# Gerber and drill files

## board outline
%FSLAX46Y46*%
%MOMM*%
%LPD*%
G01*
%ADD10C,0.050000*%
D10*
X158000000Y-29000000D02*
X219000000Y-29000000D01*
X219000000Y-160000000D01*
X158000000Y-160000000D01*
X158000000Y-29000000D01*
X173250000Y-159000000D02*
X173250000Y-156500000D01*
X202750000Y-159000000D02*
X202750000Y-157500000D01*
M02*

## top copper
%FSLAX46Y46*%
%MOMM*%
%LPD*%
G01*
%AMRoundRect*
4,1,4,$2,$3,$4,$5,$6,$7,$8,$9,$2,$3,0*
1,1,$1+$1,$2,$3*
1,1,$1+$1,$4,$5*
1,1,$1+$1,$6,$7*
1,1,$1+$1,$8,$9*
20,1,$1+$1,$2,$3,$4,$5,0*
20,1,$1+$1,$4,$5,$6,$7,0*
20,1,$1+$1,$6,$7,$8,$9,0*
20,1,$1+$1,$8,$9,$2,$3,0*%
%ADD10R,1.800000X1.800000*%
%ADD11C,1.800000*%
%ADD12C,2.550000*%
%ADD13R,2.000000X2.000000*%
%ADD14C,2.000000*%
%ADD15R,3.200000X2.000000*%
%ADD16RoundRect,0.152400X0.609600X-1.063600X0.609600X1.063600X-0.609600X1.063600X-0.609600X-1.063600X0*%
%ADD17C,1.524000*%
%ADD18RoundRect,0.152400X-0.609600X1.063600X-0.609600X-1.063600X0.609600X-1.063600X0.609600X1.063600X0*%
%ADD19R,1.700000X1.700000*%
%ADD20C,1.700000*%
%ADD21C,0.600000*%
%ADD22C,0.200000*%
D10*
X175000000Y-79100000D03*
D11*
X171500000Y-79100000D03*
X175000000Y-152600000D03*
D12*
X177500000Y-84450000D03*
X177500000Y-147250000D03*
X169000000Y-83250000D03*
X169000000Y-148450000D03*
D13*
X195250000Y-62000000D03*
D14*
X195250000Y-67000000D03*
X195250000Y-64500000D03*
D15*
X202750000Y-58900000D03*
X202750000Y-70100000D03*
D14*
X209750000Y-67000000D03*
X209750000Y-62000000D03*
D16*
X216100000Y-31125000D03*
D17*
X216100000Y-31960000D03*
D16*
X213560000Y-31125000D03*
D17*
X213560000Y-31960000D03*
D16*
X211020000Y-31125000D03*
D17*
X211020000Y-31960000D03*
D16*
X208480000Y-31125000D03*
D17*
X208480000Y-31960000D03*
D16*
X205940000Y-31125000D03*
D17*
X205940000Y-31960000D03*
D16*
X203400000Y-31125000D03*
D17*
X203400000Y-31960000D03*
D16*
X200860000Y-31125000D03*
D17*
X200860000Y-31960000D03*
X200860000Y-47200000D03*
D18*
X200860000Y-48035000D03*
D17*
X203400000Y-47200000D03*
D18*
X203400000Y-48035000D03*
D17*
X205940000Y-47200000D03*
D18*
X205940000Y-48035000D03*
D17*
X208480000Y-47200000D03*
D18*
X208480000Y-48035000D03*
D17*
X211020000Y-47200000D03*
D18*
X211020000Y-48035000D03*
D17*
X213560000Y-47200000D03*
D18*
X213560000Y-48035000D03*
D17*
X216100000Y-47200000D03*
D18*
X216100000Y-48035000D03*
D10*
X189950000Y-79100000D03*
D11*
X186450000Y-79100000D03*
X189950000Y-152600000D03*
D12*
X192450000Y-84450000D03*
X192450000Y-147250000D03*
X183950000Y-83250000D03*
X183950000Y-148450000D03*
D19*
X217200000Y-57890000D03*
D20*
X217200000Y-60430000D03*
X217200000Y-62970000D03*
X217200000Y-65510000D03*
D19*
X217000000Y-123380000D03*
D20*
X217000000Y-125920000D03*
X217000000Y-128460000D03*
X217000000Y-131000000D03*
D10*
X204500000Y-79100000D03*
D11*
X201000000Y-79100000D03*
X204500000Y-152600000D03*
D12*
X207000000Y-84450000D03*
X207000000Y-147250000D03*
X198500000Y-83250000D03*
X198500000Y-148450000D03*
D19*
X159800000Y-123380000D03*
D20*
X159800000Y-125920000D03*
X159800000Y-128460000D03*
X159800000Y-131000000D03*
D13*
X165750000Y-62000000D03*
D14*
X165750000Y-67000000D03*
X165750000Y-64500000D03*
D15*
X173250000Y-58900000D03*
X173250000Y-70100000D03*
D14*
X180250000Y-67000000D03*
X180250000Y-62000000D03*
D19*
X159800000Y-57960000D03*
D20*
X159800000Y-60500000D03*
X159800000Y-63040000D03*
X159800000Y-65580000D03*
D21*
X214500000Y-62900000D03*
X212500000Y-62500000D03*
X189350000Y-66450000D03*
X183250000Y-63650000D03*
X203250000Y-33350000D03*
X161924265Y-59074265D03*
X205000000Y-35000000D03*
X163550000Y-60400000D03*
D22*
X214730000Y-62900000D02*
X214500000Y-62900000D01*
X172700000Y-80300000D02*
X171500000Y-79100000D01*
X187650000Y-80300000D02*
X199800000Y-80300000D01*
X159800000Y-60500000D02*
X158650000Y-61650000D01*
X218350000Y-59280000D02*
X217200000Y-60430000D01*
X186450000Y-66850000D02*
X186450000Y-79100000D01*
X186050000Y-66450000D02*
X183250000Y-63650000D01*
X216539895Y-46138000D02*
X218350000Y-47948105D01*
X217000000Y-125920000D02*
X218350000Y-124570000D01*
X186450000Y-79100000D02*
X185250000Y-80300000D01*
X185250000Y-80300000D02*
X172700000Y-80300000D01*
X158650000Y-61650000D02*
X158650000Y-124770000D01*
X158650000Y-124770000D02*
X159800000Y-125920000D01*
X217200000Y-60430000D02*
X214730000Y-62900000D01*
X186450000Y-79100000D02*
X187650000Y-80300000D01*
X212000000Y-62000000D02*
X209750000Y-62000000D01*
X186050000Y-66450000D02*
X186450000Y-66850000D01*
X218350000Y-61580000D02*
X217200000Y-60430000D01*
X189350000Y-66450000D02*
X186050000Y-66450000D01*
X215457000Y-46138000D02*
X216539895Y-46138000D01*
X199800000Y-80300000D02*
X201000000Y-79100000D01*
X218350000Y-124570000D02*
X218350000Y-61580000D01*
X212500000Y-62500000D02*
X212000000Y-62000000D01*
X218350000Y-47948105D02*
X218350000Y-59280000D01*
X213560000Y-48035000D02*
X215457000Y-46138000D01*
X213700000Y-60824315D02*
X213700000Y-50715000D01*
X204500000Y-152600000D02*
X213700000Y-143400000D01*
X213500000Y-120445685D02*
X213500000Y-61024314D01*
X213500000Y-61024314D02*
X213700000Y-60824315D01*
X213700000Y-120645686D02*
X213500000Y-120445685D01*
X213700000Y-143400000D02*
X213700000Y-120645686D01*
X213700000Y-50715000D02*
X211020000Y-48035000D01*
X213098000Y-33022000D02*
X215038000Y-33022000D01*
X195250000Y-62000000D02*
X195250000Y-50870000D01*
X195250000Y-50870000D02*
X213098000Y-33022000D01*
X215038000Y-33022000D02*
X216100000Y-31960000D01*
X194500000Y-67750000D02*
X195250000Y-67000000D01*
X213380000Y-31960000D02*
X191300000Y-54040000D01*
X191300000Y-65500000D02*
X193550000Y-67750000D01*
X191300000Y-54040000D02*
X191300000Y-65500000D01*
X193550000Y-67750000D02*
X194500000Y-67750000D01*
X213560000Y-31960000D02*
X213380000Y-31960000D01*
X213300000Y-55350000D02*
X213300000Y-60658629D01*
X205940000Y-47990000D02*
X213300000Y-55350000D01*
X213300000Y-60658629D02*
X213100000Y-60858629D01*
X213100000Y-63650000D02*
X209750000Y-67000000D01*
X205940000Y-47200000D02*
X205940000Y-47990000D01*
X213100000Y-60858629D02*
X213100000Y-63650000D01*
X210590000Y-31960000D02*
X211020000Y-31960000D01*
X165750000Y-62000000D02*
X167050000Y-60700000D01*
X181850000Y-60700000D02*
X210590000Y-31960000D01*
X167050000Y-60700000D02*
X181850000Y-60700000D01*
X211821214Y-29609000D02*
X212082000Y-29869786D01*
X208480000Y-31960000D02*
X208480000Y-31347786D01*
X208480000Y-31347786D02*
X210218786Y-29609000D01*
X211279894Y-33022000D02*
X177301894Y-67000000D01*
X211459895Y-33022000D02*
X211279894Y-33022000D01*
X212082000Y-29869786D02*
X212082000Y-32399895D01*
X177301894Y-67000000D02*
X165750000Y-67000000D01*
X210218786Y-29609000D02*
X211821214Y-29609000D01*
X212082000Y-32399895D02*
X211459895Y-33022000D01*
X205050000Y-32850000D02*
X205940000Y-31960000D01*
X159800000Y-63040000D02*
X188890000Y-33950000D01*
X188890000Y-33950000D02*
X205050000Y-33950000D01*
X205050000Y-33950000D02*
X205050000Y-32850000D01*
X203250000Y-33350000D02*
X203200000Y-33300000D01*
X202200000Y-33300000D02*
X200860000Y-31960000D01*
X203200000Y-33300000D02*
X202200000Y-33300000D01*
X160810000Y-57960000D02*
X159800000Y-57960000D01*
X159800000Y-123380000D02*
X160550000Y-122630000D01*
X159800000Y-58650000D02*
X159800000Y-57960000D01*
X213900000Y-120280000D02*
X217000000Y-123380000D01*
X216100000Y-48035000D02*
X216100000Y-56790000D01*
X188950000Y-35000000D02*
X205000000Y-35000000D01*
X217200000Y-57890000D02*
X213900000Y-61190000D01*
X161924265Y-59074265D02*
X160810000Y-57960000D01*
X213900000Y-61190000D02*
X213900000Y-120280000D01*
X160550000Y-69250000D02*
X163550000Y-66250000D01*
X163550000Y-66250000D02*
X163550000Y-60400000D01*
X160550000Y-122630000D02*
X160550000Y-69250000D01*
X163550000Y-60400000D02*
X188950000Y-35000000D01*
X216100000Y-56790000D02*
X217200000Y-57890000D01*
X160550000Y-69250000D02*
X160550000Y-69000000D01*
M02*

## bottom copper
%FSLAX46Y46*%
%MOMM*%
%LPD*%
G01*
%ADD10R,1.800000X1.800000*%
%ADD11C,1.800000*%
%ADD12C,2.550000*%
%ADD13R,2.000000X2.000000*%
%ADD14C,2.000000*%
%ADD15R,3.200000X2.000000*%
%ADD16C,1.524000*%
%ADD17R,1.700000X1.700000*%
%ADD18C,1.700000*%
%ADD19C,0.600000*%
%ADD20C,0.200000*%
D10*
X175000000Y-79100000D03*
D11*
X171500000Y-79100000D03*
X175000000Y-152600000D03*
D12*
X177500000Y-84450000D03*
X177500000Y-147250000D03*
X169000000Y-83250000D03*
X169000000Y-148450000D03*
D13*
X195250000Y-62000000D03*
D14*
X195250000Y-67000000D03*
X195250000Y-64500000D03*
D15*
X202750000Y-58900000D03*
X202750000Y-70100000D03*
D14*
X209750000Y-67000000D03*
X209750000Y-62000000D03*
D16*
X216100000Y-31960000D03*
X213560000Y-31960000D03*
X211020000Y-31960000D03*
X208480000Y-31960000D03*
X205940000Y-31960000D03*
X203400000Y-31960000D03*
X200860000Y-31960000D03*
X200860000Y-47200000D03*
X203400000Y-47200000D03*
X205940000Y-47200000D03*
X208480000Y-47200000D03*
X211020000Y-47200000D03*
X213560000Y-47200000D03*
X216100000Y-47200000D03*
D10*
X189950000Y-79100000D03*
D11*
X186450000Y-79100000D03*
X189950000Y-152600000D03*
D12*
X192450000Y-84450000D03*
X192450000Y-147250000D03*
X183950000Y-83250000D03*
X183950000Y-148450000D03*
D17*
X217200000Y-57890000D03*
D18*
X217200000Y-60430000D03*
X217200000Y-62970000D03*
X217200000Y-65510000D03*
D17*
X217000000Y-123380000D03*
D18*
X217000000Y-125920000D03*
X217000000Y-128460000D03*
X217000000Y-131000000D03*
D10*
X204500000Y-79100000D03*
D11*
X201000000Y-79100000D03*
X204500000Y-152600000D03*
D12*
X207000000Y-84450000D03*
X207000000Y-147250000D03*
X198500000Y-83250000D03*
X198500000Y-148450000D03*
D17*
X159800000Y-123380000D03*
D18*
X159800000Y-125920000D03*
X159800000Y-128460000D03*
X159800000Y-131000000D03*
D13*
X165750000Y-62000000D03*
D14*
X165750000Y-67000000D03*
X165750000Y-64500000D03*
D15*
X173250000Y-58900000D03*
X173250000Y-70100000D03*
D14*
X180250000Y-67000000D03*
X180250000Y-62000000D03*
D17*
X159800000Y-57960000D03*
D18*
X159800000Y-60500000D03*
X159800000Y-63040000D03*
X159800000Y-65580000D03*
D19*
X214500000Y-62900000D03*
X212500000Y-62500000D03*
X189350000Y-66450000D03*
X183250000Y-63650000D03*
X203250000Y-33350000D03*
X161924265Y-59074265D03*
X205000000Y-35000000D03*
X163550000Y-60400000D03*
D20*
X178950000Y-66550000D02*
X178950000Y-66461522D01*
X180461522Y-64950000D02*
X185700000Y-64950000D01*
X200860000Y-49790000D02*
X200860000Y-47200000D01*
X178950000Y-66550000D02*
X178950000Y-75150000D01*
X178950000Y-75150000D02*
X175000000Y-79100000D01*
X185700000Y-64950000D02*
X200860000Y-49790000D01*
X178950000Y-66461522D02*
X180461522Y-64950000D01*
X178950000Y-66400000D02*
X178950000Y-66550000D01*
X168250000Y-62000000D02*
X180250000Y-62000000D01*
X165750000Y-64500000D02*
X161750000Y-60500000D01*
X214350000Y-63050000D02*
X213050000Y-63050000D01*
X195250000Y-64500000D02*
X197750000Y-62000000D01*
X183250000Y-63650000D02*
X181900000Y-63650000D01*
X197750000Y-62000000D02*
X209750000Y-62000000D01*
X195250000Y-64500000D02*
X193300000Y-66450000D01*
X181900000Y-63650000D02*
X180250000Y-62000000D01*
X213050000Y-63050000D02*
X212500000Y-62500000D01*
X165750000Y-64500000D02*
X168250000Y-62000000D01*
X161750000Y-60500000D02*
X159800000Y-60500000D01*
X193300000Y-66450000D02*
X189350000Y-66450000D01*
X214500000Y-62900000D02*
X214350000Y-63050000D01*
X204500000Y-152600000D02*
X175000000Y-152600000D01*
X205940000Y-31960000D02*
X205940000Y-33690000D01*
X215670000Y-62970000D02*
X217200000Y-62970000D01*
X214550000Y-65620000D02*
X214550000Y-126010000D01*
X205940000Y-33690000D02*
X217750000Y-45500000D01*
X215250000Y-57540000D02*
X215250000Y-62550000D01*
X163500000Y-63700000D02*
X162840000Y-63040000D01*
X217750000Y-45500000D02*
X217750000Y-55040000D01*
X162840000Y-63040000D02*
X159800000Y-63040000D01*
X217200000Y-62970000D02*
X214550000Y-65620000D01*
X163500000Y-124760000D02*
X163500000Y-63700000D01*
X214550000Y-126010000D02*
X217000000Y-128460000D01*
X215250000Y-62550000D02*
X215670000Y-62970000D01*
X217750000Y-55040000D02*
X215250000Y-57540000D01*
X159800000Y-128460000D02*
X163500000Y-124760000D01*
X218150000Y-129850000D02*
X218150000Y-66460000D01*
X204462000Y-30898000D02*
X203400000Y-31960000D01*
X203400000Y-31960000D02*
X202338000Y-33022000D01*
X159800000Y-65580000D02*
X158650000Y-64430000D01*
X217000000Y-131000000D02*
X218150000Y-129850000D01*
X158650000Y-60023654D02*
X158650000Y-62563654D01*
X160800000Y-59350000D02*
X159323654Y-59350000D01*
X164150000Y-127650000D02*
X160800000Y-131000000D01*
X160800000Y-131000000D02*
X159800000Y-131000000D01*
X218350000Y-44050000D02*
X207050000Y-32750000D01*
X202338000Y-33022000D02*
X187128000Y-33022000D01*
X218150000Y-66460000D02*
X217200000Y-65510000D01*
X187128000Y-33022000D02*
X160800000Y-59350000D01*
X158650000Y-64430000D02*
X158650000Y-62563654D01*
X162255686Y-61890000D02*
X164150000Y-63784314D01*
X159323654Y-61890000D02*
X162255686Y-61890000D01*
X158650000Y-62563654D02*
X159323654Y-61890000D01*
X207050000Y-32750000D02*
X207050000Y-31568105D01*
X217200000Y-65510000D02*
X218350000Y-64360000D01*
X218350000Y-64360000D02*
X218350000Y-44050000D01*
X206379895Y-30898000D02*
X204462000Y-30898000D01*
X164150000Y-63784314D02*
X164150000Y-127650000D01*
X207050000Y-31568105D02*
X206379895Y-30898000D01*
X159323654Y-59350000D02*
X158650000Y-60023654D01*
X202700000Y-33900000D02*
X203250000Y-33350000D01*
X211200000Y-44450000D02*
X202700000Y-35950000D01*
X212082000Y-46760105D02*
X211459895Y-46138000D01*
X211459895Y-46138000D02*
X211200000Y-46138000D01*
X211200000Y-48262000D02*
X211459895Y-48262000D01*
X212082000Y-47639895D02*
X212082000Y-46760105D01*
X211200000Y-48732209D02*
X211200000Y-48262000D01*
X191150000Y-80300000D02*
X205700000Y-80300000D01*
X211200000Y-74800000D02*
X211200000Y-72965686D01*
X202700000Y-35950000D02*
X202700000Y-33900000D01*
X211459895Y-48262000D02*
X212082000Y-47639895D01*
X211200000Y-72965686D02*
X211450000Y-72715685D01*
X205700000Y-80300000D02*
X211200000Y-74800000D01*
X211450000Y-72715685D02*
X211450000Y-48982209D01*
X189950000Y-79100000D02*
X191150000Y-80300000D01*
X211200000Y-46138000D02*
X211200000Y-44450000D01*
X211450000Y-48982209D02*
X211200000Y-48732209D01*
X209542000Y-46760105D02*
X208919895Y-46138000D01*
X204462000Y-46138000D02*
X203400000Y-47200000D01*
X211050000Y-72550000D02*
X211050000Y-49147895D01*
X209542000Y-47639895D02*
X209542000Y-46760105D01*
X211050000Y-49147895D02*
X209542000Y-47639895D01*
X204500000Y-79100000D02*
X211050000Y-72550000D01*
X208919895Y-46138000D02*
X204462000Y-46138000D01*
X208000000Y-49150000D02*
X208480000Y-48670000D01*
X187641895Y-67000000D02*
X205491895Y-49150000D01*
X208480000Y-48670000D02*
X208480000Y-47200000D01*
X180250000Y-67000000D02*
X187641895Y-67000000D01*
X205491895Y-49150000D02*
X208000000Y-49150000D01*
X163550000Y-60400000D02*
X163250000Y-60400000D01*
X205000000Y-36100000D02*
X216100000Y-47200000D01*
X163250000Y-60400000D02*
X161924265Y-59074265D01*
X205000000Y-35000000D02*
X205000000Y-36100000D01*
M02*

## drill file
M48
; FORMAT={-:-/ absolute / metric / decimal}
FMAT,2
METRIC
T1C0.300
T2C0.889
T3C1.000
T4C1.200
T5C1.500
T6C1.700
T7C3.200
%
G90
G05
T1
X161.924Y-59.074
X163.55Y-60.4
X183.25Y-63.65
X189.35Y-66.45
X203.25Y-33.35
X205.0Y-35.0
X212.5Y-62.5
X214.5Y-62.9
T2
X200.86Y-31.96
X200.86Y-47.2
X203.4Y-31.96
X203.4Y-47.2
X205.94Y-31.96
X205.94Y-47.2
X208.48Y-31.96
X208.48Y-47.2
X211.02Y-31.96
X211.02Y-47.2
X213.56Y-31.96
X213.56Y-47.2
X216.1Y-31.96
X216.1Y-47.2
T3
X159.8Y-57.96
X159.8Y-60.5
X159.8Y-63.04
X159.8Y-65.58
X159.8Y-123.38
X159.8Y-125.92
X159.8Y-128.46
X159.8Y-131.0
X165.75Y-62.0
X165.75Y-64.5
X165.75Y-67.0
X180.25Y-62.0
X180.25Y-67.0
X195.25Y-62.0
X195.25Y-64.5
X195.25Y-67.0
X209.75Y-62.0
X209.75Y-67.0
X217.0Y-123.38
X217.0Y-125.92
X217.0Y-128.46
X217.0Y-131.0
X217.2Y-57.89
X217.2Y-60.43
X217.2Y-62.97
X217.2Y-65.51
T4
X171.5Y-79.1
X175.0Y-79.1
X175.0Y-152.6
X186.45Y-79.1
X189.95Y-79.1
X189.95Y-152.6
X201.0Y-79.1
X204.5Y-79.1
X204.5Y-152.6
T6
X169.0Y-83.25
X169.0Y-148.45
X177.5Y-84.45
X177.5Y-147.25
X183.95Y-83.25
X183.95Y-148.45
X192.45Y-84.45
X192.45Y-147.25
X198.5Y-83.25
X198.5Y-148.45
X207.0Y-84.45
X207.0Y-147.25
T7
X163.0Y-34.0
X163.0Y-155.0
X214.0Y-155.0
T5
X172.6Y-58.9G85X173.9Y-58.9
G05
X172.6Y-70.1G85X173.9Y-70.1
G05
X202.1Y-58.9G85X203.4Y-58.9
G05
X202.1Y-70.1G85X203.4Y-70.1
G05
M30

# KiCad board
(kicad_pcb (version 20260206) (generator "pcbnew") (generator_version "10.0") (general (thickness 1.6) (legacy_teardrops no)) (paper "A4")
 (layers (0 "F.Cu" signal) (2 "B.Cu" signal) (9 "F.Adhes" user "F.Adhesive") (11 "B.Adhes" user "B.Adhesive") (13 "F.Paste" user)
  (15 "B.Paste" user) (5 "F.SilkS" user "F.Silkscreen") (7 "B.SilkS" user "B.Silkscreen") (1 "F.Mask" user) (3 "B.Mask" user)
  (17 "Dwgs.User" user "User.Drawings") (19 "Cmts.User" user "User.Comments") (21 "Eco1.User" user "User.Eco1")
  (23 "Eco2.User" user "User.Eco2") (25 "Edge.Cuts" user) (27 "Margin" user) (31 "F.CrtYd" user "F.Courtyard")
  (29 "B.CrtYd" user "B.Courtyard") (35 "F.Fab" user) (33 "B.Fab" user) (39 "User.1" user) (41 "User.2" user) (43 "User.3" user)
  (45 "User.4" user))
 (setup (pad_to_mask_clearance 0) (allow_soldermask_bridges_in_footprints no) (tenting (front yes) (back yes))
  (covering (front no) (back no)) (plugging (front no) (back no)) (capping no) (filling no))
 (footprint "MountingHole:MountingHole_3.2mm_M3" (layer "F.Cu") (at 163 34)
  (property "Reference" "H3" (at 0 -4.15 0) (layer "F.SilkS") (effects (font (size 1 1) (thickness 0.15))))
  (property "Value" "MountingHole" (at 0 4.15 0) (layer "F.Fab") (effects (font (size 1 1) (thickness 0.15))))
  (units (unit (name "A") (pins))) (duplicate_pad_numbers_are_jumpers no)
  (pad "" np_thru_hole circle (at 0 0) (size 3.2 3.2) (drill 3.2) (layers "*.Cu" "*.Mask")))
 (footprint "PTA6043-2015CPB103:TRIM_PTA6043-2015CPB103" (layer "F.Cu") (at 173.25 115.85 -90)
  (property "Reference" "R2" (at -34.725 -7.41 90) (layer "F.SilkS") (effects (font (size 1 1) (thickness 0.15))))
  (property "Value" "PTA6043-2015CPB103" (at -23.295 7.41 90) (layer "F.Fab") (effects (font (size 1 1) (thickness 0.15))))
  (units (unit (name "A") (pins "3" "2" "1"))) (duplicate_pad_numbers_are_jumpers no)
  (pad "1" thru_hole rect (at -36.75 -1.75 270) (size 1.8 1.8) (drill 1.2) (layers "*.Cu" "*.Mask") (remove_unused_layers no) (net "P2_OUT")
   (solder_mask_margin 0.102))
  (pad "2" thru_hole circle (at -36.75 1.75 270) (size 1.8 1.8) (drill 1.2) (layers "*.Cu" "*.Mask") (remove_unused_layers no) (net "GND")
   (solder_mask_margin 0.102))
  (pad "3" thru_hole circle (at 36.75 -1.75 270) (size 1.8 1.8) (drill 1.2) (layers "*.Cu" "*.Mask") (remove_unused_layers no) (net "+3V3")
   (solder_mask_margin 0.102))
  (pad "SH1" thru_hole circle (at -31.4 -4.25 270) (size 2.55 2.55) (drill 1.7) (layers "*.Cu" "*.Mask") (remove_unused_layers no)
   (solder_mask_margin 0.102))
  (pad "SH2" thru_hole circle (at 31.4 -4.25 270) (size 2.55 2.55) (drill 1.7) (layers "*.Cu" "*.Mask") (remove_unused_layers no)
   (solder_mask_margin 0.102))
  (pad "SH3" thru_hole circle (at -32.6 4.25 270) (size 2.55 2.55) (drill 1.7) (layers "*.Cu" "*.Mask") (remove_unused_layers no)
   (solder_mask_margin 0.102))
  (pad "SH4" thru_hole circle (at 32.6 4.25 270) (size 2.55 2.55) (drill 1.7) (layers "*.Cu" "*.Mask") (remove_unused_layers no)
   (solder_mask_margin 0.102)))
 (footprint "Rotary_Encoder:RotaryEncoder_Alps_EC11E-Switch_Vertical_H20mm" (layer "F.Cu") (at 195.25 62)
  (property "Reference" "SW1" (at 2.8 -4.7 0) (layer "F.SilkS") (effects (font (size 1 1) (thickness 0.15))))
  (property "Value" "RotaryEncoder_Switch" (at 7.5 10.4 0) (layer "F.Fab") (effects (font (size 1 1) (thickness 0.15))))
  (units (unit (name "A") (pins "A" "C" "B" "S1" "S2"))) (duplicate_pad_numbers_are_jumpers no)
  (pad "A" thru_hole rect (at 0 0) (size 2 2) (drill 1) (layers "*.Cu" "*.Mask") (remove_unused_layers no) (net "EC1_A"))
  (pad "B" thru_hole circle (at 0 5) (size 2 2) (drill 1) (layers "*.Cu" "*.Mask") (remove_unused_layers no) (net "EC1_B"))
  (pad "C" thru_hole circle (at 0 2.5) (size 2 2) (drill 1) (layers "*.Cu" "*.Mask") (remove_unused_layers no) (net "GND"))
  (pad "MP" thru_hole rect (at 7.5 -3.1) (size 3.2 2) (drill oval 2.8 1.5) (layers "*.Cu" "*.Mask") (remove_unused_layers no))
  (pad "MP" thru_hole rect (at 7.5 8.1) (size 3.2 2) (drill oval 2.8 1.5) (layers "*.Cu" "*.Mask") (remove_unused_layers no))
  (pad "S1" thru_hole circle (at 14.5 5) (size 2 2) (drill 1) (layers "*.Cu" "*.Mask") (remove_unused_layers no) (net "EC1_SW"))
  (pad "S2" thru_hole circle (at 14.5 0) (size 2 2) (drill 1) (layers "*.Cu" "*.Mask") (remove_unused_layers no) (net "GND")))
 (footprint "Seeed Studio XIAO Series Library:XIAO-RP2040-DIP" (layer "F.Cu") (at 208.48 39.58)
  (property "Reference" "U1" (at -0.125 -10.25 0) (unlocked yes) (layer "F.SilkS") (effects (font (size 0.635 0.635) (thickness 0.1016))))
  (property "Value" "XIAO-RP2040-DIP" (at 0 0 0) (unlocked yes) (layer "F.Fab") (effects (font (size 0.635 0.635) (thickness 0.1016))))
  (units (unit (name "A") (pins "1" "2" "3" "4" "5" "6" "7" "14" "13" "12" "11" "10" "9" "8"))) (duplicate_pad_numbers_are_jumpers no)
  (pad "1" smd roundrect (at 7.62 -8.455 90) (size 2.432 1.524) (layers "F.Cu" "F.Mask") (roundrect_rratio 0.1) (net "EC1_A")
   (thermal_bridge_angle 45))
  (pad "1" thru_hole circle (at 7.62 -7.62 90) (size 1.524 1.524) (drill 0.889) (layers "*.Cu" "*.Mask") (remove_unused_layers no)
   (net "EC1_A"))
  (pad "2" smd roundrect (at 5.08 -8.455 90) (size 2.432 1.524) (layers "F.Cu" "F.Mask") (roundrect_rratio 0.1) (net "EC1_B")
   (thermal_bridge_angle 45))
  (pad "2" thru_hole circle (at 5.08 -7.62 90) (size 1.524 1.524) (drill 0.889) (layers "*.Cu" "*.Mask") (remove_unused_layers no)
   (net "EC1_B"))
  (pad "3" smd roundrect (at 2.54 -8.455 90) (size 2.432 1.524) (layers "F.Cu" "F.Mask") (roundrect_rratio 0.1) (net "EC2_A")
   (thermal_bridge_angle 45))
  (pad "3" thru_hole circle (at 2.54 -7.62 90) (size 1.524 1.524) (drill 0.889) (layers "*.Cu" "*.Mask") (remove_unused_layers no)
   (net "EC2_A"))
  (pad "4" smd roundrect (at 0 -8.455 90) (size 2.432 1.524) (layers "F.Cu" "F.Mask") (roundrect_rratio 0.1) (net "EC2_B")
   (thermal_bridge_angle 45))
  (pad "4" thru_hole circle (at 0 -7.62 90) (size 1.524 1.524) (drill 0.889) (layers "*.Cu" "*.Mask") (remove_unused_layers no)
   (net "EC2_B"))
  (pad "5" smd roundrect (at -2.54 -8.455 90) (size 2.432 1.524) (layers "F.Cu" "F.Mask") (roundrect_rratio 0.1) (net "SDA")
   (thermal_bridge_angle 45))
  (pad "5" thru_hole circle (at -2.54 -7.62 90) (size 1.524 1.524) (drill 0.889) (layers "*.Cu" "*.Mask") (remove_unused_layers no)
   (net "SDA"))
  (pad "6" smd roundrect (at -5.08 -8.455 90) (size 2.432 1.524) (layers "F.Cu" "F.Mask") (roundrect_rratio 0.1) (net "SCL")
   (thermal_bridge_angle 45))
  (pad "6" thru_hole circle (at -5.08 -7.62 90) (size 1.524 1.524) (drill 0.889) (layers "*.Cu" "*.Mask") (remove_unused_layers no)
   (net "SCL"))
  (pad "7" smd roundrect (at -7.62 -8.455 90) (size 2.432 1.524) (layers "F.Cu" "F.Mask") (roundrect_rratio 0.1) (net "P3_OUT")
   (thermal_bridge_angle 45))
  (pad "7" thru_hole circle (at -7.62 -7.62 90) (size 1.524 1.524) (drill 0.889) (layers "*.Cu" "*.Mask") (remove_unused_layers no)
   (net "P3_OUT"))
  (pad "8" thru_hole circle (at -7.62 7.62 270) (size 1.524 1.524) (drill 0.889) (layers "*.Cu" "*.Mask") (remove_unused_layers no)
   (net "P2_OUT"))
  (pad "8" smd roundrect (at -7.62 8.455 270) (size 2.432 1.524) (layers "F.Cu" "F.Mask") (roundrect_rratio 0.1) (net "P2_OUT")
   (thermal_bridge_angle 45))
  (pad "9" thru_hole circle (at -5.08 7.62 270) (size 1.524 1.524) (drill 0.889) (layers "*.Cu" "*.Mask") (remove_unused_layers no)
   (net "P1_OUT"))
  (pad "9" smd roundrect (at -5.08 8.455 270) (size 2.432 1.524) (layers "F.Cu" "F.Mask") (roundrect_rratio 0.1) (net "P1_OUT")
   (thermal_bridge_angle 45))
  (pad "10" thru_hole circle (at -2.54 7.62 270) (size 1.524 1.524) (drill 0.889) (layers "*.Cu" "*.Mask") (remove_unused_layers no)
   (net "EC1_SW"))
  (pad "10" smd roundrect (at -2.54 8.455 270) (size 2.432 1.524) (layers "F.Cu" "F.Mask") (roundrect_rratio 0.1) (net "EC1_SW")
   (thermal_bridge_angle 45))
  (pad "11" thru_hole circle (at 0 7.62 270) (size 1.524 1.524) (drill 0.889) (layers "*.Cu" "*.Mask") (remove_unused_layers no)
   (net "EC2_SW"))
  (pad "11" smd roundrect (at 0 8.455 270) (size 2.432 1.524) (layers "F.Cu" "F.Mask") (roundrect_rratio 0.1) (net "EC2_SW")
   (thermal_bridge_angle 45))
  (pad "12" thru_hole circle (at 2.54 7.62 270) (size 1.524 1.524) (drill 0.889) (layers "*.Cu" "*.Mask") (remove_unused_layers no)
   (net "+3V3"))
  (pad "12" smd roundrect (at 2.54 8.455 270) (size 2.432 1.524) (layers "F.Cu" "F.Mask") (roundrect_rratio 0.1) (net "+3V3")
   (thermal_bridge_angle 45))
  (pad "13" thru_hole circle (at 5.08 7.62 270) (size 1.524 1.524) (drill 0.889) (layers "*.Cu" "*.Mask") (remove_unused_layers no)
   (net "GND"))
  (pad "13" smd roundrect (at 5.08 8.455 270) (size 2.432 1.524) (layers "F.Cu" "F.Mask") (roundrect_rratio 0.1) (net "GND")
   (thermal_bridge_angle 45))
  (pad "14" thru_hole circle (at 7.62 7.62 270) (size 1.524 1.524) (drill 0.889) (layers "*.Cu" "*.Mask") (remove_unused_layers no)
   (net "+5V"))
  (pad "14" smd roundrect (at 7.62 8.455 270) (size 2.432 1.524) (layers "F.Cu" "F.Mask") (roundrect_rratio 0.1) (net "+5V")
   (thermal_bridge_angle 45)))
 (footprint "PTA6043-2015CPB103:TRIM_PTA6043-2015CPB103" (layer "F.Cu") (at 188.2 115.85 -90)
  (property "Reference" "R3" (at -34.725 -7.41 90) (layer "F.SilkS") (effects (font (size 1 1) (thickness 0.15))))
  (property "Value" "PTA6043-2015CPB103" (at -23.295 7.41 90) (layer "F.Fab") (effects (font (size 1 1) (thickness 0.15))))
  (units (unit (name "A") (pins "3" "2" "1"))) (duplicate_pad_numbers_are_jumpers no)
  (pad "1" thru_hole rect (at -36.75 -1.75 270) (size 1.8 1.8) (drill 1.2) (layers "*.Cu" "*.Mask") (remove_unused_layers no) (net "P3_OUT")
   (solder_mask_margin 0.102))
  (pad "2" thru_hole circle (at -36.75 1.75 270) (size 1.8 1.8) (drill 1.2) (layers "*.Cu" "*.Mask") (remove_unused_layers no) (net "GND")
   (solder_mask_margin 0.102))
  (pad "3" thru_hole circle (at 36.75 -1.75 270) (size 1.8 1.8) (drill 1.2) (layers "*.Cu" "*.Mask") (remove_unused_layers no) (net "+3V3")
   (solder_mask_margin 0.102))
  (pad "SH1" thru_hole circle (at -31.4 -4.25 270) (size 2.55 2.55) (drill 1.7) (layers "*.Cu" "*.Mask") (remove_unused_layers no)
   (solder_mask_margin 0.102))
  (pad "SH2" thru_hole circle (at 31.4 -4.25 270) (size 2.55 2.55) (drill 1.7) (layers "*.Cu" "*.Mask") (remove_unused_layers no)
   (solder_mask_margin 0.102))
  (pad "SH3" thru_hole circle (at -32.6 4.25 270) (size 2.55 2.55) (drill 1.7) (layers "*.Cu" "*.Mask") (remove_unused_layers no)
   (solder_mask_margin 0.102))
  (pad "SH4" thru_hole circle (at 32.6 4.25 270) (size 2.55 2.55) (drill 1.7) (layers "*.Cu" "*.Mask") (remove_unused_layers no)
   (solder_mask_margin 0.102)))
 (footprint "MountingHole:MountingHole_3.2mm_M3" (layer "F.Cu") (at 163 155)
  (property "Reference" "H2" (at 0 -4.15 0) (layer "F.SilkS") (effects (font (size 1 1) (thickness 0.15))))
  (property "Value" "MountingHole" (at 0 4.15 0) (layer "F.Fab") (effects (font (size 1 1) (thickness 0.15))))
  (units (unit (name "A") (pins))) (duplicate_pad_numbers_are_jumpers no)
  (pad "" np_thru_hole circle (at 0 0) (size 3.2 3.2) (drill 3.2) (layers "*.Cu" "*.Mask")))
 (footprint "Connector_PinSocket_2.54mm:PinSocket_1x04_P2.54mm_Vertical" (layer "F.Cu") (at 217.2 57.89)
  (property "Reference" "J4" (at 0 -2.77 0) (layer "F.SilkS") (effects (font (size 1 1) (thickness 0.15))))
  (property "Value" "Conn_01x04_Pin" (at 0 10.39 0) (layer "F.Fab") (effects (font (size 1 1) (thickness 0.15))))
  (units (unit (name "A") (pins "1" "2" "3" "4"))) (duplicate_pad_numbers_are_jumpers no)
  (pad "1" thru_hole rect (at 0 0) (size 1.7 1.7) (drill 1) (layers "*.Cu" "*.Mask") (remove_unused_layers no) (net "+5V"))
  (pad "2" thru_hole circle (at 0 2.54) (size 1.7 1.7) (drill 1) (layers "*.Cu" "*.Mask") (remove_unused_layers no) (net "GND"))
  (pad "3" thru_hole circle (at 0 5.08) (size 1.7 1.7) (drill 1) (layers "*.Cu" "*.Mask") (remove_unused_layers no) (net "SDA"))
  (pad "4" thru_hole circle (at 0 7.62) (size 1.7 1.7) (drill 1) (layers "*.Cu" "*.Mask") (remove_unused_layers no) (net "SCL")))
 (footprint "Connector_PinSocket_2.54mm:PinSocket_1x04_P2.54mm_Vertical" (layer "F.Cu") (at 217 123.38)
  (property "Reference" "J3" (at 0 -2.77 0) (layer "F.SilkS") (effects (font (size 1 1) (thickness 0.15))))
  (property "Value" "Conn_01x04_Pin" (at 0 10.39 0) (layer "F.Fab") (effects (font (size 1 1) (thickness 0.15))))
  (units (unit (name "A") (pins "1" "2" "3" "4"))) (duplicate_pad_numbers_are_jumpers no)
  (pad "1" thru_hole rect (at 0 0) (size 1.7 1.7) (drill 1) (layers "*.Cu" "*.Mask") (remove_unused_layers no) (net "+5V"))
  (pad "2" thru_hole circle (at 0 2.54) (size 1.7 1.7) (drill 1) (layers "*.Cu" "*.Mask") (remove_unused_layers no) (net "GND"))
  (pad "3" thru_hole circle (at 0 5.08) (size 1.7 1.7) (drill 1) (layers "*.Cu" "*.Mask") (remove_unused_layers no) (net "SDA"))
  (pad "4" thru_hole circle (at 0 7.62) (size 1.7 1.7) (drill 1) (layers "*.Cu" "*.Mask") (remove_unused_layers no) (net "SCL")))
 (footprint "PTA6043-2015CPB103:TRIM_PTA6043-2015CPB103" (layer "F.Cu") (at 202.75 115.85 -90)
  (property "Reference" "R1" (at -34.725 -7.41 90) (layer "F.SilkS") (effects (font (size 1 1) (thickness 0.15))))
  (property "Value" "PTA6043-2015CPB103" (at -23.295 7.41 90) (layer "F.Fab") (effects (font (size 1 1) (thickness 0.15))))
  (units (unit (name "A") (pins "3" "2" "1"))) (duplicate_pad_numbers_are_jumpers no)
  (pad "1" thru_hole rect (at -36.75 -1.75 270) (size 1.8 1.8) (drill 1.2) (layers "*.Cu" "*.Mask") (remove_unused_layers no) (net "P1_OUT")
   (solder_mask_margin 0.102))
  (pad "2" thru_hole circle (at -36.75 1.75 270) (size 1.8 1.8) (drill 1.2) (layers "*.Cu" "*.Mask") (remove_unused_layers no) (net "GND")
   (solder_mask_margin 0.102))
  (pad "3" thru_hole circle (at 36.75 -1.75 270) (size 1.8 1.8) (drill 1.2) (layers "*.Cu" "*.Mask") (remove_unused_layers no) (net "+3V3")
   (solder_mask_margin 0.102))
  (pad "SH1" thru_hole circle (at -31.4 -4.25 270) (size 2.55 2.55) (drill 1.7) (layers "*.Cu" "*.Mask") (remove_unused_layers no)
   (solder_mask_margin 0.102))
  (pad "SH2" thru_hole circle (at 31.4 -4.25 270) (size 2.55 2.55) (drill 1.7) (layers "*.Cu" "*.Mask") (remove_unused_layers no)
   (solder_mask_margin 0.102))
  (pad "SH3" thru_hole circle (at -32.6 4.25 270) (size 2.55 2.55) (drill 1.7) (layers "*.Cu" "*.Mask") (remove_unused_layers no)
   (solder_mask_margin 0.102))
  (pad "SH4" thru_hole circle (at 32.6 4.25 270) (size 2.55 2.55) (drill 1.7) (layers "*.Cu" "*.Mask") (remove_unused_layers no)
   (solder_mask_margin 0.102)))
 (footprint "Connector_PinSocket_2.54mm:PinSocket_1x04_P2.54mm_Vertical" (layer "F.Cu") (at 159.8 123.38)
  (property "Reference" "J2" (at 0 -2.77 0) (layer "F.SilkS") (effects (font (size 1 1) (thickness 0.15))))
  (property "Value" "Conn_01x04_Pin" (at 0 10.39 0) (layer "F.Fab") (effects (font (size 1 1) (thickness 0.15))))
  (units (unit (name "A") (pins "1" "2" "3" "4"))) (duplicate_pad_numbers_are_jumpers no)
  (pad "1" thru_hole rect (at 0 0) (size 1.7 1.7) (drill 1) (layers "*.Cu" "*.Mask") (remove_unused_layers no) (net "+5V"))
  (pad "2" thru_hole circle (at 0 2.54) (size 1.7 1.7) (drill 1) (layers "*.Cu" "*.Mask") (remove_unused_layers no) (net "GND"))
  (pad "3" thru_hole circle (at 0 5.08) (size 1.7 1.7) (drill 1) (layers "*.Cu" "*.Mask") (remove_unused_layers no) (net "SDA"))
  (pad "4" thru_hole circle (at 0 7.62) (size 1.7 1.7) (drill 1) (layers "*.Cu" "*.Mask") (remove_unused_layers no) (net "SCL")))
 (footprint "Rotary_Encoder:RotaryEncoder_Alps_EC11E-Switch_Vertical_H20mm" (layer "F.Cu") (at 165.75 62)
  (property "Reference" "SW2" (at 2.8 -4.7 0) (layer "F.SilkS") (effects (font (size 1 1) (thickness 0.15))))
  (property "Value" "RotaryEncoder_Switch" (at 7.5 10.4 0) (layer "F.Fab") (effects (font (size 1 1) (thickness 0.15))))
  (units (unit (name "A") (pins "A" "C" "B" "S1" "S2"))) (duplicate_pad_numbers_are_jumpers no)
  (pad "A" thru_hole rect (at 0 0) (size 2 2) (drill 1) (layers "*.Cu" "*.Mask") (remove_unused_layers no) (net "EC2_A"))
  (pad "B" thru_hole circle (at 0 5) (size 2 2) (drill 1) (layers "*.Cu" "*.Mask") (remove_unused_layers no) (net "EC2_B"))
  (pad "C" thru_hole circle (at 0 2.5) (size 2 2) (drill 1) (layers "*.Cu" "*.Mask") (remove_unused_layers no) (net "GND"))
  (pad "MP" thru_hole rect (at 7.5 -3.1) (size 3.2 2) (drill oval 2.8 1.5) (layers "*.Cu" "*.Mask") (remove_unused_layers no))
  (pad "MP" thru_hole rect (at 7.5 8.1) (size 3.2 2) (drill oval 2.8 1.5) (layers "*.Cu" "*.Mask") (remove_unused_layers no))
  (pad "S1" thru_hole circle (at 14.5 5) (size 2 2) (drill 1) (layers "*.Cu" "*.Mask") (remove_unused_layers no) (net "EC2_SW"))
  (pad "S2" thru_hole circle (at 14.5 0) (size 2 2) (drill 1) (layers "*.Cu" "*.Mask") (remove_unused_layers no) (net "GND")))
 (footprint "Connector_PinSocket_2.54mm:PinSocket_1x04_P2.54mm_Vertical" (layer "F.Cu") (at 159.8 57.96)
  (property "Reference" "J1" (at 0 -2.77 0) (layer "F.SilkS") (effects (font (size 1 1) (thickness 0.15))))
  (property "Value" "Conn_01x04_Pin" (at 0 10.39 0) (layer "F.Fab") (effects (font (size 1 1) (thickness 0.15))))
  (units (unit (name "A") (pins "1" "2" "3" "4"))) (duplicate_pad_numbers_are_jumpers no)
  (pad "1" thru_hole rect (at 0 0) (size 1.7 1.7) (drill 1) (layers "*.Cu" "*.Mask") (remove_unused_layers no) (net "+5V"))
  (pad "2" thru_hole circle (at 0 2.54) (size 1.7 1.7) (drill 1) (layers "*.Cu" "*.Mask") (remove_unused_layers no) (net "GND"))
  (pad "3" thru_hole circle (at 0 5.08) (size 1.7 1.7) (drill 1) (layers "*.Cu" "*.Mask") (remove_unused_layers no) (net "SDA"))
  (pad "4" thru_hole circle (at 0 7.62) (size 1.7 1.7) (drill 1) (layers "*.Cu" "*.Mask") (remove_unused_layers no) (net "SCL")))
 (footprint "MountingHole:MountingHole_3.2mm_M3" (layer "F.Cu") (at 214 155)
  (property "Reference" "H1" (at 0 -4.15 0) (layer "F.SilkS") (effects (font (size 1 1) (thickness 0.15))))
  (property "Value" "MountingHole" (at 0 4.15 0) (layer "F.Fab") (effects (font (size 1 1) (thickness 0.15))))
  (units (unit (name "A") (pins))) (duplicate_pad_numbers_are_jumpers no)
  (pad "" np_thru_hole circle (at 0 0) (size 3.2 3.2) (drill 3.2) (layers "*.Cu" "*.Mask")))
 (gr_rect (start 158 29) (end 219 160) (stroke (width 0.05) (type default)) (fill no) (layer "Edge.Cuts"))
 (gr_line (start 173.25 159) (end 173.25 156.5) (stroke (width 0.05) (type default)) (layer "Edge.Cuts"))
 (gr_line (start 202.75 159) (end 202.75 157.5) (stroke (width 0.05) (type default)) (layer "Edge.Cuts"))
 (segment (start 178.95 66.55) (end 178.95 66.461522) (width 0.2) (layer "B.Cu") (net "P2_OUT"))
 (segment (start 180.461522 64.95) (end 185.7 64.95) (width 0.2) (layer "B.Cu") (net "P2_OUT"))
 (segment (start 200.86 49.79) (end 200.86 47.2) (width 0.2) (layer "B.Cu") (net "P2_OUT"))
 (segment (start 178.95 66.55) (end 178.95 75.15) (width 0.2) (layer "B.Cu") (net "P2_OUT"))
 (segment (start 178.95 75.15) (end 175 79.1) (width 0.2) (layer "B.Cu") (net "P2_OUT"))
 (segment (start 185.7 64.95) (end 200.86 49.79) (width 0.2) (layer "B.Cu") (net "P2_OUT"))
 (segment (start 178.95 66.461522) (end 180.461522 64.95) (width 0.2) (layer "B.Cu") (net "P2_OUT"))
 (segment (start 178.95 66.4) (end 178.95 66.55) (width 0.2) (layer "B.Cu") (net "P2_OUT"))
 (segment (start 214.73 62.9) (end 214.5 62.9) (width 0.2) (layer "F.Cu") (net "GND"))
 (segment (start 172.7 80.3) (end 171.5 79.1) (width 0.2) (layer "F.Cu") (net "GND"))
 (segment (start 187.65 80.3) (end 199.8 80.3) (width 0.2) (layer "F.Cu") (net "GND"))
 (segment (start 159.8 60.5) (end 158.65 61.65) (width 0.2) (layer "F.Cu") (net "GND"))
 (segment (start 218.35 59.28) (end 217.2 60.43) (width 0.2) (layer "F.Cu") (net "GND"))
 (segment (start 186.45 66.85) (end 186.45 79.1) (width 0.2) (layer "F.Cu") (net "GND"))
 (segment (start 186.05 66.45) (end 183.25 63.65) (width 0.2) (layer "F.Cu") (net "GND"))
 (segment (start 216.539895 46.138) (end 218.35 47.948105) (width 0.2) (layer "F.Cu") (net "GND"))
 (segment (start 217 125.92) (end 218.35 124.57) (width 0.2) (layer "F.Cu") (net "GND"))
 (segment (start 186.45 79.1) (end 185.25 80.3) (width 0.2) (layer "F.Cu") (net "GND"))
 (segment (start 185.25 80.3) (end 172.7 80.3) (width 0.2) (layer "F.Cu") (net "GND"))
 (segment (start 158.65 61.65) (end 158.65 124.77) (width 0.2) (layer "F.Cu") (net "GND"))
 (segment (start 158.65 124.77) (end 159.8 125.92) (width 0.2) (layer "F.Cu") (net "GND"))
 (segment (start 217.2 60.43) (end 214.73 62.9) (width 0.2) (layer "F.Cu") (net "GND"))
 (segment (start 186.45 79.1) (end 187.65 80.3) (width 0.2) (layer "F.Cu") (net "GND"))
 (segment (start 212 62) (end 209.75 62) (width 0.2) (layer "F.Cu") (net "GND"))
 (segment (start 186.05 66.45) (end 186.45 66.85) (width 0.2) (layer "F.Cu") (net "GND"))
 (segment (start 218.35 61.58) (end 217.2 60.43) (width 0.2) (layer "F.Cu") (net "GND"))
 (segment (start 189.35 66.45) (end 186.05 66.45) (width 0.2) (layer "F.Cu") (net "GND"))
 (segment (start 215.457 46.138) (end 216.539895 46.138) (width 0.2) (layer "F.Cu") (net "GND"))
 (segment (start 199.8 80.3) (end 201 79.1) (width 0.2) (layer "F.Cu") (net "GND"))
 (segment (start 218.35 124.57) (end 218.35 61.58) (width 0.2) (layer "F.Cu") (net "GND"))
 (segment (start 212.5 62.5) (end 212 62) (width 0.2) (layer "F.Cu") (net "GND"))
 (segment (start 218.35 47.948105) (end 218.35 59.28) (width 0.2) (layer "F.Cu") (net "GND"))
 (segment (start 213.56 48.035) (end 215.457 46.138) (width 0.2) (layer "F.Cu") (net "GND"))
 (via (at 214.5 62.9) (size 0.6) (drill 0.3) (layers "F.Cu" "B.Cu") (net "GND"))
 (via (at 212.5 62.5) (size 0.6) (drill 0.3) (layers "F.Cu" "B.Cu") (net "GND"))
 (via (at 189.35 66.45) (size 0.6) (drill 0.3) (layers "F.Cu" "B.Cu") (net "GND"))
 (via (at 183.25 63.65) (size 0.6) (drill 0.3) (layers "F.Cu" "B.Cu") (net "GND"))
 (segment (start 168.25 62) (end 180.25 62) (width 0.2) (layer "B.Cu") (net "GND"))
 (segment (start 165.75 64.5) (end 161.75 60.5) (width 0.2) (layer "B.Cu") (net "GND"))
 (segment (start 214.35 63.05) (end 213.05 63.05) (width 0.2) (layer "B.Cu") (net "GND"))
 (segment (start 195.25 64.5) (end 197.75 62) (width 0.2) (layer "B.Cu") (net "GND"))
 (segment (start 183.25 63.65) (end 181.9 63.65) (width 0.2) (layer "B.Cu") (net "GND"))
 (segment (start 197.75 62) (end 209.75 62) (width 0.2) (layer "B.Cu") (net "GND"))
 (segment (start 195.25 64.5) (end 193.3 66.45) (width 0.2) (layer "B.Cu") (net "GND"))
 (segment (start 181.9 63.65) (end 180.25 62) (width 0.2) (layer "B.Cu") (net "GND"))
 (segment (start 213.05 63.05) (end 212.5 62.5) (width 0.2) (layer "B.Cu") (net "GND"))
 (segment (start 165.75 64.5) (end 168.25 62) (width 0.2) (layer "B.Cu") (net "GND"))
 (segment (start 161.75 60.5) (end 159.8 60.5) (width 0.2) (layer "B.Cu") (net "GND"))
 (segment (start 193.3 66.45) (end 189.35 66.45) (width 0.2) (layer "B.Cu") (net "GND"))
 (segment (start 214.5 62.9) (end 214.35 63.05) (width 0.2) (layer "B.Cu") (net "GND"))
 (segment (start 213.7 60.824315) (end 213.7 50.715) (width 0.2) (layer "F.Cu") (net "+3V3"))
 (segment (start 204.5 152.6) (end 213.7 143.4) (width 0.2) (layer "F.Cu") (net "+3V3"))
 (segment (start 213.5 120.445685) (end 213.5 61.024314) (width 0.2) (layer "F.Cu") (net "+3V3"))
 (segment (start 213.5 61.024314) (end 213.7 60.824315) (width 0.2) (layer "F.Cu") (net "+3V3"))
 (segment (start 213.7 120.645686) (end 213.5 120.445685) (width 0.2) (layer "F.Cu") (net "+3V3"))
 (segment (start 213.7 143.4) (end 213.7 120.645686) (width 0.2) (layer "F.Cu") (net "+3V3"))
 (segment (start 213.7 50.715) (end 211.02 48.035) (width 0.2) (layer "F.Cu") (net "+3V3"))
 (segment (start 204.5 152.6) (end 175 152.6) (width 0.2) (layer "B.Cu") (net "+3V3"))
 (segment (start 213.098 33.022) (end 215.038 33.022) (width 0.2) (layer "F.Cu") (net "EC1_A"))
 (segment (start 195.25 62) (end 195.25 50.87) (width 0.2) (layer "F.Cu") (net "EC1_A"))
 (segment (start 195.25 50.87) (end 213.098 33.022) (width 0.2) (layer "F.Cu") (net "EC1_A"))
 (segment (start 215.038 33.022) (end 216.1 31.96) (width 0.2) (layer "F.Cu") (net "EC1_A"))
 (segment (start 194.5 67.75) (end 195.25 67) (width 0.2) (layer "F.Cu") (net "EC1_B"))
 (segment (start 213.38 31.96) (end 191.3 54.04) (width 0.2) (layer "F.Cu") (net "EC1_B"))
 (segment (start 191.3 65.5) (end 193.55 67.75) (width 0.2) (layer "F.Cu") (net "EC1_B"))
 (segment (start 191.3 54.04) (end 191.3 65.5) (width 0.2) (layer "F.Cu") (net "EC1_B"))
 (segment (start 193.55 67.75) (end 194.5 67.75) (width 0.2) (layer "F.Cu") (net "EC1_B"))
 (segment (start 213.56 31.96) (end 213.38 31.96) (width 0.2) (layer "F.Cu") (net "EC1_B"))
 (segment (start 213.3 55.35) (end 213.3 60.658629) (width 0.2) (layer "F.Cu") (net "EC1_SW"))
 (segment (start 205.94 47.99) (end 213.3 55.35) (width 0.2) (layer "F.Cu") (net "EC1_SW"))
 (segment (start 213.3 60.658629) (end 213.1 60.858629) (width 0.2) (layer "F.Cu") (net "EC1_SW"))
 (segment (start 213.1 63.65) (end 209.75 67) (width 0.2) (layer "F.Cu") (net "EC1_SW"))
 (segment (start 205.94 47.2) (end 205.94 47.99) (width 0.2) (layer "F.Cu") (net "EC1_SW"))
 (segment (start 213.1 60.858629) (end 213.1 63.65) (width 0.2) (layer "F.Cu") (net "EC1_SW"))
 (segment (start 210.59 31.96) (end 211.02 31.96) (width 0.2) (layer "F.Cu") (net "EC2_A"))
 (segment (start 165.75 62) (end 167.05 60.7) (width 0.2) (layer "F.Cu") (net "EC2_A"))
 (segment (start 181.85 60.7) (end 210.59 31.96) (width 0.2) (layer "F.Cu") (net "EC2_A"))
 (segment (start 167.05 60.7) (end 181.85 60.7) (width 0.2) (layer "F.Cu") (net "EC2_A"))
 (segment (start 211.821214 29.609) (end 212.082 29.869786) (width 0.2) (layer "F.Cu") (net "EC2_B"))
 (segment (start 208.48 31.96) (end 208.48 31.347786) (width 0.2) (layer "F.Cu") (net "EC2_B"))
 (segment (start 208.48 31.347786) (end 210.218786 29.609) (width 0.2) (layer "F.Cu") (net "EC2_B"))
 (segment (start 211.279894 33.022) (end 177.301894 67) (width 0.2) (layer "F.Cu") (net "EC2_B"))
 (segment (start 211.459895 33.022) (end 211.279894 33.022) (width 0.2) (layer "F.Cu") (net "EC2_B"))
 (segment (start 212.082 29.869786) (end 212.082 32.399895) (width 0.2) (layer "F.Cu") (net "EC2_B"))
 (segment (start 177.301894 67) (end 165.75 67) (width 0.2) (layer "F.Cu") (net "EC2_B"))
 (segment (start 210.218786 29.609) (end 211.821214 29.609) (width 0.2) (layer "F.Cu") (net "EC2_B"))
 (segment (start 212.082 32.399895) (end 211.459895 33.022) (width 0.2) (layer "F.Cu") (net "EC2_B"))
 (segment (start 205.05 32.85) (end 205.94 31.96) (width 0.2) (layer "F.Cu") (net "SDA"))
 (segment (start 159.8 63.04) (end 188.89 33.95) (width 0.2) (layer "F.Cu") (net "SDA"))
 (segment (start 188.89 33.95) (end 205.05 33.95) (width 0.2) (layer "F.Cu") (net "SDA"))
 (segment (start 205.05 33.95) (end 205.05 32.85) (width 0.2) (layer "F.Cu") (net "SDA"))
 (segment (start 205.94 31.96) (end 205.94 33.69) (width 0.2) (layer "B.Cu") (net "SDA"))
 (segment (start 215.67 62.97) (end 217.2 62.97) (width 0.2) (layer "B.Cu") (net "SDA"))
 (segment (start 214.55 65.62) (end 214.55 126.01) (width 0.2) (layer "B.Cu") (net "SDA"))
 (segment (start 205.94 33.69) (end 217.75 45.5) (width 0.2) (layer "B.Cu") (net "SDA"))
 (segment (start 215.25 57.54) (end 215.25 62.55) (width 0.2) (layer "B.Cu") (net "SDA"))
 (segment (start 163.5 63.7) (end 162.84 63.04) (width 0.2) (layer "B.Cu") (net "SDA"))
 (segment (start 217.75 45.5) (end 217.75 55.04) (width 0.2) (layer "B.Cu") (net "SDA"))
 (segment (start 162.84 63.04) (end 159.8 63.04) (width 0.2) (layer "B.Cu") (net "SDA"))
 (segment (start 217.2 62.97) (end 214.55 65.62) (width 0.2) (layer "B.Cu") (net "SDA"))
 (segment (start 163.5 124.76) (end 163.5 63.7) (width 0.2) (layer "B.Cu") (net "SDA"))
 (segment (start 214.55 126.01) (end 217 128.46) (width 0.2) (layer "B.Cu") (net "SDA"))
 (segment (start 215.25 62.55) (end 215.67 62.97) (width 0.2) (layer "B.Cu") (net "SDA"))
 (segment (start 217.75 55.04) (end 215.25 57.54) (width 0.2) (layer "B.Cu") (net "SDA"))
 (segment (start 159.8 128.46) (end 163.5 124.76) (width 0.2) (layer "B.Cu") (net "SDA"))
 (segment (start 218.15 129.85) (end 218.15 66.46) (width 0.2) (layer "B.Cu") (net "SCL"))
 (segment (start 204.462 30.898) (end 203.4 31.96) (width 0.2) (layer "B.Cu") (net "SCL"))
 (segment (start 203.4 31.96) (end 202.338 33.022) (width 0.2) (layer "B.Cu") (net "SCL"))
 (segment (start 159.8 65.58) (end 158.65 64.43) (width 0.2) (layer "B.Cu") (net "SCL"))
 (segment (start 217 131) (end 218.15 129.85) (width 0.2) (layer "B.Cu") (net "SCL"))
 (segment (start 158.65 60.023654) (end 158.65 62.563654) (width 0.2) (layer "B.Cu") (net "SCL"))
 (segment (start 160.8 59.35) (end 159.323654 59.35) (width 0.2) (layer "B.Cu") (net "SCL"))
 (segment (start 164.15 127.65) (end 160.8 131) (width 0.2) (layer "B.Cu") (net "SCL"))
 (segment (start 160.8 131) (end 159.8 131) (width 0.2) (layer "B.Cu") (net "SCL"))
 (segment (start 218.35 44.05) (end 207.05 32.75) (width 0.2) (layer "B.Cu") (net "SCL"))
 (segment (start 202.338 33.022) (end 187.128 33.022) (width 0.2) (layer "B.Cu") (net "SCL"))
 (segment (start 218.15 66.46) (end 217.2 65.51) (width 0.2) (layer "B.Cu") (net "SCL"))
 (segment (start 187.128 33.022) (end 160.8 59.35) (width 0.2) (layer "B.Cu") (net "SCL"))
 (segment (start 158.65 64.43) (end 158.65 62.563654) (width 0.2) (layer "B.Cu") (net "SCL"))
 (segment (start 162.255686 61.89) (end 164.15 63.784314) (width 0.2) (layer "B.Cu") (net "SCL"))
 (segment (start 159.323654 61.89) (end 162.255686 61.89) (width 0.2) (layer "B.Cu") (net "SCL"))
 (segment (start 158.65 62.563654) (end 159.323654 61.89) (width 0.2) (layer "B.Cu") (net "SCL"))
 (segment (start 207.05 32.75) (end 207.05 31.568105) (width 0.2) (layer "B.Cu") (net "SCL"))
 (segment (start 217.2 65.51) (end 218.35 64.36) (width 0.2) (layer "B.Cu") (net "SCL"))
 (segment (start 218.35 64.36) (end 218.35 44.05) (width 0.2) (layer "B.Cu") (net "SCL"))
 (segment (start 206.379895 30.898) (end 204.462 30.898) (width 0.2) (layer "B.Cu") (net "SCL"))
 (segment (start 164.15 63.784314) (end 164.15 127.65) (width 0.2) (layer "B.Cu") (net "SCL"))
 (segment (start 207.05 31.568105) (end 206.379895 30.898) (width 0.2) (layer "B.Cu") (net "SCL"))
 (segment (start 159.323654 59.35) (end 158.65 60.023654) (width 0.2) (layer "B.Cu") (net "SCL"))
 (segment (start 203.25 33.35) (end 203.2 33.3) (width 0.2) (layer "F.Cu") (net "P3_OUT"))
 (segment (start 202.2 33.3) (end 200.86 31.96) (width 0.2) (layer "F.Cu") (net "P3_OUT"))
 (segment (start 203.2 33.3) (end 202.2 33.3) (width 0.2) (layer "F.Cu") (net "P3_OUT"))
 (via (at 203.25 33.35) (size 0.6) (drill 0.3) (layers "F.Cu" "B.Cu") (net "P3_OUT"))
 (segment (start 202.7 33.9) (end 203.25 33.35) (width 0.2) (layer "B.Cu") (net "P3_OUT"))
 (segment (start 211.2 44.45) (end 202.7 35.95) (width 0.2) (layer "B.Cu") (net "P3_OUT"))
 (segment (start 212.082 46.760105) (end 211.459895 46.138) (width 0.2) (layer "B.Cu") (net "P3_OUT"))
 (segment (start 211.459895 46.138) (end 211.2 46.138) (width 0.2) (layer "B.Cu") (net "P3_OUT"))
 (segment (start 211.2 48.262) (end 211.459895 48.262) (width 0.2) (layer "B.Cu") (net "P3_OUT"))
 (segment (start 212.082 47.639895) (end 212.082 46.760105) (width 0.2) (layer "B.Cu") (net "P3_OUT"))
 (segment (start 211.2 48.732209) (end 211.2 48.262) (width 0.2) (layer "B.Cu") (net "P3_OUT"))
 (segment (start 191.15 80.3) (end 205.7 80.3) (width 0.2) (layer "B.Cu") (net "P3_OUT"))
 (segment (start 211.2 74.8) (end 211.2 72.965686) (width 0.2) (layer "B.Cu") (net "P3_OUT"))
 (segment (start 202.7 35.95) (end 202.7 33.9) (width 0.2) (layer "B.Cu") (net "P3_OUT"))
 (segment (start 211.459895 48.262) (end 212.082 47.639895) (width 0.2) (layer "B.Cu") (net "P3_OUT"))
 (segment (start 211.2 72.965686) (end 211.45 72.715685) (width 0.2) (layer "B.Cu") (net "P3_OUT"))
 (segment (start 205.7 80.3) (end 211.2 74.8) (width 0.2) (layer "B.Cu") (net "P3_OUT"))
 (segment (start 211.45 72.715685) (end 211.45 48.982209) (width 0.2) (layer "B.Cu") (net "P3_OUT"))
 (segment (start 189.95 79.1) (end 191.15 80.3) (width 0.2) (layer "B.Cu") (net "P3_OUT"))
 (segment (start 211.2 46.138) (end 211.2 44.45) (width 0.2) (layer "B.Cu") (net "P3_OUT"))
 (segment (start 211.45 48.982209) (end 211.2 48.732209) (width 0.2) (layer "B.Cu") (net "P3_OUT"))
 (segment (start 209.542 46.760105) (end 208.919895 46.138) (width 0.2) (layer "B.Cu") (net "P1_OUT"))
 (segment (start 204.462 46.138) (end 203.4 47.2) (width 0.2) (layer "B.Cu") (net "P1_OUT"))
 (segment (start 211.05 72.55) (end 211.05 49.147895) (width 0.2) (layer "B.Cu") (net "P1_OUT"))
 (segment (start 209.542 47.639895) (end 209.542 46.760105) (width 0.2) (layer "B.Cu") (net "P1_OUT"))
 (segment (start 211.05 49.147895) (end 209.542 47.639895) (width 0.2) (layer "B.Cu") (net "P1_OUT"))
 (segment (start 204.5 79.1) (end 211.05 72.55) (width 0.2) (layer "B.Cu") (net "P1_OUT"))
 (segment (start 208.919895 46.138) (end 204.462 46.138) (width 0.2) (layer "B.Cu") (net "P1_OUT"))
 (segment (start 208 49.15) (end 208.48 48.67) (width 0.2) (layer "B.Cu") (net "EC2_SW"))
 (segment (start 187.641895 67) (end 205.491895 49.15) (width 0.2) (layer "B.Cu") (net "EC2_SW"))
 (segment (start 208.48 48.67) (end 208.48 47.2) (width 0.2) (layer "B.Cu") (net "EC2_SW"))
 (segment (start 180.25 67) (end 187.641895 67) (width 0.2) (layer "B.Cu") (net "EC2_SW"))
 (segment (start 205.491895 49.15) (end 208 49.15) (width 0.2) (layer "B.Cu") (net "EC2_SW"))
 (segment (start 160.81 57.96) (end 159.8 57.96) (width 0.2) (layer "F.Cu") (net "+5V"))
 (segment (start 159.8 123.38) (end 160.55 122.63) (width 0.2) (layer "F.Cu") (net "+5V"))
 (segment (start 159.8 58.65) (end 159.8 57.96) (width 0.2) (layer "F.Cu") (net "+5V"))
 (segment (start 213.9 120.28) (end 217 123.38) (width 0.2) (layer "F.Cu") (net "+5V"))
 (segment (start 216.1 48.035) (end 216.1 56.79) (width 0.2) (layer "F.Cu") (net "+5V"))
 (segment (start 188.95 35) (end 205 35) (width 0.2) (layer "F.Cu") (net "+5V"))
 (segment (start 217.2 57.89) (end 213.9 61.19) (width 0.2) (layer "F.Cu") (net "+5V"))
 (segment (start 161.924265 59.074265) (end 160.81 57.96) (width 0.2) (layer "F.Cu") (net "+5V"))
 (segment (start 213.9 61.19) (end 213.9 120.28) (width 0.2) (layer "F.Cu") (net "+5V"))
 (segment (start 160.55 69.25) (end 163.55 66.25) (width 0.2) (layer "F.Cu") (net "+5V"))
 (segment (start 163.55 66.25) (end 163.55 60.4) (width 0.2) (layer "F.Cu") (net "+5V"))
 (segment (start 160.55 122.63) (end 160.55 69.25) (width 0.2) (layer "F.Cu") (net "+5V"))
 (segment (start 163.55 60.4) (end 188.95 35) (width 0.2) (layer "F.Cu") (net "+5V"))
 (segment (start 216.1 56.79) (end 217.2 57.89) (width 0.2) (layer "F.Cu") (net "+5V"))
 (segment (start 160.55 69.25) (end 160.55 69) (width 0.2) (layer "F.Cu") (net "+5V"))
 (via (at 161.924265 59.074265) (size 0.6) (drill 0.3) (layers "F.Cu" "B.Cu") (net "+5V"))
 (via (at 205 35) (size 0.6) (drill 0.3) (layers "F.Cu" "B.Cu") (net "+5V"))
 (via (at 163.55 60.4) (size 0.6) (drill 0.3) (layers "F.Cu" "B.Cu") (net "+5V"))
 (segment (start 163.55 60.4) (end 163.25 60.4) (width 0.2) (layer "B.Cu") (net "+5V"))
 (segment (start 205 36.1) (end 216.1 47.2) (width 0.2) (layer "B.Cu") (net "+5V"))
 (segment (start 163.25 60.4) (end 161.924265 59.074265) (width 0.2) (layer "B.Cu") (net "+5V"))
 (segment (start 205 35) (end 205 36.1) (width 0.2) (layer "B.Cu") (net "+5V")))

